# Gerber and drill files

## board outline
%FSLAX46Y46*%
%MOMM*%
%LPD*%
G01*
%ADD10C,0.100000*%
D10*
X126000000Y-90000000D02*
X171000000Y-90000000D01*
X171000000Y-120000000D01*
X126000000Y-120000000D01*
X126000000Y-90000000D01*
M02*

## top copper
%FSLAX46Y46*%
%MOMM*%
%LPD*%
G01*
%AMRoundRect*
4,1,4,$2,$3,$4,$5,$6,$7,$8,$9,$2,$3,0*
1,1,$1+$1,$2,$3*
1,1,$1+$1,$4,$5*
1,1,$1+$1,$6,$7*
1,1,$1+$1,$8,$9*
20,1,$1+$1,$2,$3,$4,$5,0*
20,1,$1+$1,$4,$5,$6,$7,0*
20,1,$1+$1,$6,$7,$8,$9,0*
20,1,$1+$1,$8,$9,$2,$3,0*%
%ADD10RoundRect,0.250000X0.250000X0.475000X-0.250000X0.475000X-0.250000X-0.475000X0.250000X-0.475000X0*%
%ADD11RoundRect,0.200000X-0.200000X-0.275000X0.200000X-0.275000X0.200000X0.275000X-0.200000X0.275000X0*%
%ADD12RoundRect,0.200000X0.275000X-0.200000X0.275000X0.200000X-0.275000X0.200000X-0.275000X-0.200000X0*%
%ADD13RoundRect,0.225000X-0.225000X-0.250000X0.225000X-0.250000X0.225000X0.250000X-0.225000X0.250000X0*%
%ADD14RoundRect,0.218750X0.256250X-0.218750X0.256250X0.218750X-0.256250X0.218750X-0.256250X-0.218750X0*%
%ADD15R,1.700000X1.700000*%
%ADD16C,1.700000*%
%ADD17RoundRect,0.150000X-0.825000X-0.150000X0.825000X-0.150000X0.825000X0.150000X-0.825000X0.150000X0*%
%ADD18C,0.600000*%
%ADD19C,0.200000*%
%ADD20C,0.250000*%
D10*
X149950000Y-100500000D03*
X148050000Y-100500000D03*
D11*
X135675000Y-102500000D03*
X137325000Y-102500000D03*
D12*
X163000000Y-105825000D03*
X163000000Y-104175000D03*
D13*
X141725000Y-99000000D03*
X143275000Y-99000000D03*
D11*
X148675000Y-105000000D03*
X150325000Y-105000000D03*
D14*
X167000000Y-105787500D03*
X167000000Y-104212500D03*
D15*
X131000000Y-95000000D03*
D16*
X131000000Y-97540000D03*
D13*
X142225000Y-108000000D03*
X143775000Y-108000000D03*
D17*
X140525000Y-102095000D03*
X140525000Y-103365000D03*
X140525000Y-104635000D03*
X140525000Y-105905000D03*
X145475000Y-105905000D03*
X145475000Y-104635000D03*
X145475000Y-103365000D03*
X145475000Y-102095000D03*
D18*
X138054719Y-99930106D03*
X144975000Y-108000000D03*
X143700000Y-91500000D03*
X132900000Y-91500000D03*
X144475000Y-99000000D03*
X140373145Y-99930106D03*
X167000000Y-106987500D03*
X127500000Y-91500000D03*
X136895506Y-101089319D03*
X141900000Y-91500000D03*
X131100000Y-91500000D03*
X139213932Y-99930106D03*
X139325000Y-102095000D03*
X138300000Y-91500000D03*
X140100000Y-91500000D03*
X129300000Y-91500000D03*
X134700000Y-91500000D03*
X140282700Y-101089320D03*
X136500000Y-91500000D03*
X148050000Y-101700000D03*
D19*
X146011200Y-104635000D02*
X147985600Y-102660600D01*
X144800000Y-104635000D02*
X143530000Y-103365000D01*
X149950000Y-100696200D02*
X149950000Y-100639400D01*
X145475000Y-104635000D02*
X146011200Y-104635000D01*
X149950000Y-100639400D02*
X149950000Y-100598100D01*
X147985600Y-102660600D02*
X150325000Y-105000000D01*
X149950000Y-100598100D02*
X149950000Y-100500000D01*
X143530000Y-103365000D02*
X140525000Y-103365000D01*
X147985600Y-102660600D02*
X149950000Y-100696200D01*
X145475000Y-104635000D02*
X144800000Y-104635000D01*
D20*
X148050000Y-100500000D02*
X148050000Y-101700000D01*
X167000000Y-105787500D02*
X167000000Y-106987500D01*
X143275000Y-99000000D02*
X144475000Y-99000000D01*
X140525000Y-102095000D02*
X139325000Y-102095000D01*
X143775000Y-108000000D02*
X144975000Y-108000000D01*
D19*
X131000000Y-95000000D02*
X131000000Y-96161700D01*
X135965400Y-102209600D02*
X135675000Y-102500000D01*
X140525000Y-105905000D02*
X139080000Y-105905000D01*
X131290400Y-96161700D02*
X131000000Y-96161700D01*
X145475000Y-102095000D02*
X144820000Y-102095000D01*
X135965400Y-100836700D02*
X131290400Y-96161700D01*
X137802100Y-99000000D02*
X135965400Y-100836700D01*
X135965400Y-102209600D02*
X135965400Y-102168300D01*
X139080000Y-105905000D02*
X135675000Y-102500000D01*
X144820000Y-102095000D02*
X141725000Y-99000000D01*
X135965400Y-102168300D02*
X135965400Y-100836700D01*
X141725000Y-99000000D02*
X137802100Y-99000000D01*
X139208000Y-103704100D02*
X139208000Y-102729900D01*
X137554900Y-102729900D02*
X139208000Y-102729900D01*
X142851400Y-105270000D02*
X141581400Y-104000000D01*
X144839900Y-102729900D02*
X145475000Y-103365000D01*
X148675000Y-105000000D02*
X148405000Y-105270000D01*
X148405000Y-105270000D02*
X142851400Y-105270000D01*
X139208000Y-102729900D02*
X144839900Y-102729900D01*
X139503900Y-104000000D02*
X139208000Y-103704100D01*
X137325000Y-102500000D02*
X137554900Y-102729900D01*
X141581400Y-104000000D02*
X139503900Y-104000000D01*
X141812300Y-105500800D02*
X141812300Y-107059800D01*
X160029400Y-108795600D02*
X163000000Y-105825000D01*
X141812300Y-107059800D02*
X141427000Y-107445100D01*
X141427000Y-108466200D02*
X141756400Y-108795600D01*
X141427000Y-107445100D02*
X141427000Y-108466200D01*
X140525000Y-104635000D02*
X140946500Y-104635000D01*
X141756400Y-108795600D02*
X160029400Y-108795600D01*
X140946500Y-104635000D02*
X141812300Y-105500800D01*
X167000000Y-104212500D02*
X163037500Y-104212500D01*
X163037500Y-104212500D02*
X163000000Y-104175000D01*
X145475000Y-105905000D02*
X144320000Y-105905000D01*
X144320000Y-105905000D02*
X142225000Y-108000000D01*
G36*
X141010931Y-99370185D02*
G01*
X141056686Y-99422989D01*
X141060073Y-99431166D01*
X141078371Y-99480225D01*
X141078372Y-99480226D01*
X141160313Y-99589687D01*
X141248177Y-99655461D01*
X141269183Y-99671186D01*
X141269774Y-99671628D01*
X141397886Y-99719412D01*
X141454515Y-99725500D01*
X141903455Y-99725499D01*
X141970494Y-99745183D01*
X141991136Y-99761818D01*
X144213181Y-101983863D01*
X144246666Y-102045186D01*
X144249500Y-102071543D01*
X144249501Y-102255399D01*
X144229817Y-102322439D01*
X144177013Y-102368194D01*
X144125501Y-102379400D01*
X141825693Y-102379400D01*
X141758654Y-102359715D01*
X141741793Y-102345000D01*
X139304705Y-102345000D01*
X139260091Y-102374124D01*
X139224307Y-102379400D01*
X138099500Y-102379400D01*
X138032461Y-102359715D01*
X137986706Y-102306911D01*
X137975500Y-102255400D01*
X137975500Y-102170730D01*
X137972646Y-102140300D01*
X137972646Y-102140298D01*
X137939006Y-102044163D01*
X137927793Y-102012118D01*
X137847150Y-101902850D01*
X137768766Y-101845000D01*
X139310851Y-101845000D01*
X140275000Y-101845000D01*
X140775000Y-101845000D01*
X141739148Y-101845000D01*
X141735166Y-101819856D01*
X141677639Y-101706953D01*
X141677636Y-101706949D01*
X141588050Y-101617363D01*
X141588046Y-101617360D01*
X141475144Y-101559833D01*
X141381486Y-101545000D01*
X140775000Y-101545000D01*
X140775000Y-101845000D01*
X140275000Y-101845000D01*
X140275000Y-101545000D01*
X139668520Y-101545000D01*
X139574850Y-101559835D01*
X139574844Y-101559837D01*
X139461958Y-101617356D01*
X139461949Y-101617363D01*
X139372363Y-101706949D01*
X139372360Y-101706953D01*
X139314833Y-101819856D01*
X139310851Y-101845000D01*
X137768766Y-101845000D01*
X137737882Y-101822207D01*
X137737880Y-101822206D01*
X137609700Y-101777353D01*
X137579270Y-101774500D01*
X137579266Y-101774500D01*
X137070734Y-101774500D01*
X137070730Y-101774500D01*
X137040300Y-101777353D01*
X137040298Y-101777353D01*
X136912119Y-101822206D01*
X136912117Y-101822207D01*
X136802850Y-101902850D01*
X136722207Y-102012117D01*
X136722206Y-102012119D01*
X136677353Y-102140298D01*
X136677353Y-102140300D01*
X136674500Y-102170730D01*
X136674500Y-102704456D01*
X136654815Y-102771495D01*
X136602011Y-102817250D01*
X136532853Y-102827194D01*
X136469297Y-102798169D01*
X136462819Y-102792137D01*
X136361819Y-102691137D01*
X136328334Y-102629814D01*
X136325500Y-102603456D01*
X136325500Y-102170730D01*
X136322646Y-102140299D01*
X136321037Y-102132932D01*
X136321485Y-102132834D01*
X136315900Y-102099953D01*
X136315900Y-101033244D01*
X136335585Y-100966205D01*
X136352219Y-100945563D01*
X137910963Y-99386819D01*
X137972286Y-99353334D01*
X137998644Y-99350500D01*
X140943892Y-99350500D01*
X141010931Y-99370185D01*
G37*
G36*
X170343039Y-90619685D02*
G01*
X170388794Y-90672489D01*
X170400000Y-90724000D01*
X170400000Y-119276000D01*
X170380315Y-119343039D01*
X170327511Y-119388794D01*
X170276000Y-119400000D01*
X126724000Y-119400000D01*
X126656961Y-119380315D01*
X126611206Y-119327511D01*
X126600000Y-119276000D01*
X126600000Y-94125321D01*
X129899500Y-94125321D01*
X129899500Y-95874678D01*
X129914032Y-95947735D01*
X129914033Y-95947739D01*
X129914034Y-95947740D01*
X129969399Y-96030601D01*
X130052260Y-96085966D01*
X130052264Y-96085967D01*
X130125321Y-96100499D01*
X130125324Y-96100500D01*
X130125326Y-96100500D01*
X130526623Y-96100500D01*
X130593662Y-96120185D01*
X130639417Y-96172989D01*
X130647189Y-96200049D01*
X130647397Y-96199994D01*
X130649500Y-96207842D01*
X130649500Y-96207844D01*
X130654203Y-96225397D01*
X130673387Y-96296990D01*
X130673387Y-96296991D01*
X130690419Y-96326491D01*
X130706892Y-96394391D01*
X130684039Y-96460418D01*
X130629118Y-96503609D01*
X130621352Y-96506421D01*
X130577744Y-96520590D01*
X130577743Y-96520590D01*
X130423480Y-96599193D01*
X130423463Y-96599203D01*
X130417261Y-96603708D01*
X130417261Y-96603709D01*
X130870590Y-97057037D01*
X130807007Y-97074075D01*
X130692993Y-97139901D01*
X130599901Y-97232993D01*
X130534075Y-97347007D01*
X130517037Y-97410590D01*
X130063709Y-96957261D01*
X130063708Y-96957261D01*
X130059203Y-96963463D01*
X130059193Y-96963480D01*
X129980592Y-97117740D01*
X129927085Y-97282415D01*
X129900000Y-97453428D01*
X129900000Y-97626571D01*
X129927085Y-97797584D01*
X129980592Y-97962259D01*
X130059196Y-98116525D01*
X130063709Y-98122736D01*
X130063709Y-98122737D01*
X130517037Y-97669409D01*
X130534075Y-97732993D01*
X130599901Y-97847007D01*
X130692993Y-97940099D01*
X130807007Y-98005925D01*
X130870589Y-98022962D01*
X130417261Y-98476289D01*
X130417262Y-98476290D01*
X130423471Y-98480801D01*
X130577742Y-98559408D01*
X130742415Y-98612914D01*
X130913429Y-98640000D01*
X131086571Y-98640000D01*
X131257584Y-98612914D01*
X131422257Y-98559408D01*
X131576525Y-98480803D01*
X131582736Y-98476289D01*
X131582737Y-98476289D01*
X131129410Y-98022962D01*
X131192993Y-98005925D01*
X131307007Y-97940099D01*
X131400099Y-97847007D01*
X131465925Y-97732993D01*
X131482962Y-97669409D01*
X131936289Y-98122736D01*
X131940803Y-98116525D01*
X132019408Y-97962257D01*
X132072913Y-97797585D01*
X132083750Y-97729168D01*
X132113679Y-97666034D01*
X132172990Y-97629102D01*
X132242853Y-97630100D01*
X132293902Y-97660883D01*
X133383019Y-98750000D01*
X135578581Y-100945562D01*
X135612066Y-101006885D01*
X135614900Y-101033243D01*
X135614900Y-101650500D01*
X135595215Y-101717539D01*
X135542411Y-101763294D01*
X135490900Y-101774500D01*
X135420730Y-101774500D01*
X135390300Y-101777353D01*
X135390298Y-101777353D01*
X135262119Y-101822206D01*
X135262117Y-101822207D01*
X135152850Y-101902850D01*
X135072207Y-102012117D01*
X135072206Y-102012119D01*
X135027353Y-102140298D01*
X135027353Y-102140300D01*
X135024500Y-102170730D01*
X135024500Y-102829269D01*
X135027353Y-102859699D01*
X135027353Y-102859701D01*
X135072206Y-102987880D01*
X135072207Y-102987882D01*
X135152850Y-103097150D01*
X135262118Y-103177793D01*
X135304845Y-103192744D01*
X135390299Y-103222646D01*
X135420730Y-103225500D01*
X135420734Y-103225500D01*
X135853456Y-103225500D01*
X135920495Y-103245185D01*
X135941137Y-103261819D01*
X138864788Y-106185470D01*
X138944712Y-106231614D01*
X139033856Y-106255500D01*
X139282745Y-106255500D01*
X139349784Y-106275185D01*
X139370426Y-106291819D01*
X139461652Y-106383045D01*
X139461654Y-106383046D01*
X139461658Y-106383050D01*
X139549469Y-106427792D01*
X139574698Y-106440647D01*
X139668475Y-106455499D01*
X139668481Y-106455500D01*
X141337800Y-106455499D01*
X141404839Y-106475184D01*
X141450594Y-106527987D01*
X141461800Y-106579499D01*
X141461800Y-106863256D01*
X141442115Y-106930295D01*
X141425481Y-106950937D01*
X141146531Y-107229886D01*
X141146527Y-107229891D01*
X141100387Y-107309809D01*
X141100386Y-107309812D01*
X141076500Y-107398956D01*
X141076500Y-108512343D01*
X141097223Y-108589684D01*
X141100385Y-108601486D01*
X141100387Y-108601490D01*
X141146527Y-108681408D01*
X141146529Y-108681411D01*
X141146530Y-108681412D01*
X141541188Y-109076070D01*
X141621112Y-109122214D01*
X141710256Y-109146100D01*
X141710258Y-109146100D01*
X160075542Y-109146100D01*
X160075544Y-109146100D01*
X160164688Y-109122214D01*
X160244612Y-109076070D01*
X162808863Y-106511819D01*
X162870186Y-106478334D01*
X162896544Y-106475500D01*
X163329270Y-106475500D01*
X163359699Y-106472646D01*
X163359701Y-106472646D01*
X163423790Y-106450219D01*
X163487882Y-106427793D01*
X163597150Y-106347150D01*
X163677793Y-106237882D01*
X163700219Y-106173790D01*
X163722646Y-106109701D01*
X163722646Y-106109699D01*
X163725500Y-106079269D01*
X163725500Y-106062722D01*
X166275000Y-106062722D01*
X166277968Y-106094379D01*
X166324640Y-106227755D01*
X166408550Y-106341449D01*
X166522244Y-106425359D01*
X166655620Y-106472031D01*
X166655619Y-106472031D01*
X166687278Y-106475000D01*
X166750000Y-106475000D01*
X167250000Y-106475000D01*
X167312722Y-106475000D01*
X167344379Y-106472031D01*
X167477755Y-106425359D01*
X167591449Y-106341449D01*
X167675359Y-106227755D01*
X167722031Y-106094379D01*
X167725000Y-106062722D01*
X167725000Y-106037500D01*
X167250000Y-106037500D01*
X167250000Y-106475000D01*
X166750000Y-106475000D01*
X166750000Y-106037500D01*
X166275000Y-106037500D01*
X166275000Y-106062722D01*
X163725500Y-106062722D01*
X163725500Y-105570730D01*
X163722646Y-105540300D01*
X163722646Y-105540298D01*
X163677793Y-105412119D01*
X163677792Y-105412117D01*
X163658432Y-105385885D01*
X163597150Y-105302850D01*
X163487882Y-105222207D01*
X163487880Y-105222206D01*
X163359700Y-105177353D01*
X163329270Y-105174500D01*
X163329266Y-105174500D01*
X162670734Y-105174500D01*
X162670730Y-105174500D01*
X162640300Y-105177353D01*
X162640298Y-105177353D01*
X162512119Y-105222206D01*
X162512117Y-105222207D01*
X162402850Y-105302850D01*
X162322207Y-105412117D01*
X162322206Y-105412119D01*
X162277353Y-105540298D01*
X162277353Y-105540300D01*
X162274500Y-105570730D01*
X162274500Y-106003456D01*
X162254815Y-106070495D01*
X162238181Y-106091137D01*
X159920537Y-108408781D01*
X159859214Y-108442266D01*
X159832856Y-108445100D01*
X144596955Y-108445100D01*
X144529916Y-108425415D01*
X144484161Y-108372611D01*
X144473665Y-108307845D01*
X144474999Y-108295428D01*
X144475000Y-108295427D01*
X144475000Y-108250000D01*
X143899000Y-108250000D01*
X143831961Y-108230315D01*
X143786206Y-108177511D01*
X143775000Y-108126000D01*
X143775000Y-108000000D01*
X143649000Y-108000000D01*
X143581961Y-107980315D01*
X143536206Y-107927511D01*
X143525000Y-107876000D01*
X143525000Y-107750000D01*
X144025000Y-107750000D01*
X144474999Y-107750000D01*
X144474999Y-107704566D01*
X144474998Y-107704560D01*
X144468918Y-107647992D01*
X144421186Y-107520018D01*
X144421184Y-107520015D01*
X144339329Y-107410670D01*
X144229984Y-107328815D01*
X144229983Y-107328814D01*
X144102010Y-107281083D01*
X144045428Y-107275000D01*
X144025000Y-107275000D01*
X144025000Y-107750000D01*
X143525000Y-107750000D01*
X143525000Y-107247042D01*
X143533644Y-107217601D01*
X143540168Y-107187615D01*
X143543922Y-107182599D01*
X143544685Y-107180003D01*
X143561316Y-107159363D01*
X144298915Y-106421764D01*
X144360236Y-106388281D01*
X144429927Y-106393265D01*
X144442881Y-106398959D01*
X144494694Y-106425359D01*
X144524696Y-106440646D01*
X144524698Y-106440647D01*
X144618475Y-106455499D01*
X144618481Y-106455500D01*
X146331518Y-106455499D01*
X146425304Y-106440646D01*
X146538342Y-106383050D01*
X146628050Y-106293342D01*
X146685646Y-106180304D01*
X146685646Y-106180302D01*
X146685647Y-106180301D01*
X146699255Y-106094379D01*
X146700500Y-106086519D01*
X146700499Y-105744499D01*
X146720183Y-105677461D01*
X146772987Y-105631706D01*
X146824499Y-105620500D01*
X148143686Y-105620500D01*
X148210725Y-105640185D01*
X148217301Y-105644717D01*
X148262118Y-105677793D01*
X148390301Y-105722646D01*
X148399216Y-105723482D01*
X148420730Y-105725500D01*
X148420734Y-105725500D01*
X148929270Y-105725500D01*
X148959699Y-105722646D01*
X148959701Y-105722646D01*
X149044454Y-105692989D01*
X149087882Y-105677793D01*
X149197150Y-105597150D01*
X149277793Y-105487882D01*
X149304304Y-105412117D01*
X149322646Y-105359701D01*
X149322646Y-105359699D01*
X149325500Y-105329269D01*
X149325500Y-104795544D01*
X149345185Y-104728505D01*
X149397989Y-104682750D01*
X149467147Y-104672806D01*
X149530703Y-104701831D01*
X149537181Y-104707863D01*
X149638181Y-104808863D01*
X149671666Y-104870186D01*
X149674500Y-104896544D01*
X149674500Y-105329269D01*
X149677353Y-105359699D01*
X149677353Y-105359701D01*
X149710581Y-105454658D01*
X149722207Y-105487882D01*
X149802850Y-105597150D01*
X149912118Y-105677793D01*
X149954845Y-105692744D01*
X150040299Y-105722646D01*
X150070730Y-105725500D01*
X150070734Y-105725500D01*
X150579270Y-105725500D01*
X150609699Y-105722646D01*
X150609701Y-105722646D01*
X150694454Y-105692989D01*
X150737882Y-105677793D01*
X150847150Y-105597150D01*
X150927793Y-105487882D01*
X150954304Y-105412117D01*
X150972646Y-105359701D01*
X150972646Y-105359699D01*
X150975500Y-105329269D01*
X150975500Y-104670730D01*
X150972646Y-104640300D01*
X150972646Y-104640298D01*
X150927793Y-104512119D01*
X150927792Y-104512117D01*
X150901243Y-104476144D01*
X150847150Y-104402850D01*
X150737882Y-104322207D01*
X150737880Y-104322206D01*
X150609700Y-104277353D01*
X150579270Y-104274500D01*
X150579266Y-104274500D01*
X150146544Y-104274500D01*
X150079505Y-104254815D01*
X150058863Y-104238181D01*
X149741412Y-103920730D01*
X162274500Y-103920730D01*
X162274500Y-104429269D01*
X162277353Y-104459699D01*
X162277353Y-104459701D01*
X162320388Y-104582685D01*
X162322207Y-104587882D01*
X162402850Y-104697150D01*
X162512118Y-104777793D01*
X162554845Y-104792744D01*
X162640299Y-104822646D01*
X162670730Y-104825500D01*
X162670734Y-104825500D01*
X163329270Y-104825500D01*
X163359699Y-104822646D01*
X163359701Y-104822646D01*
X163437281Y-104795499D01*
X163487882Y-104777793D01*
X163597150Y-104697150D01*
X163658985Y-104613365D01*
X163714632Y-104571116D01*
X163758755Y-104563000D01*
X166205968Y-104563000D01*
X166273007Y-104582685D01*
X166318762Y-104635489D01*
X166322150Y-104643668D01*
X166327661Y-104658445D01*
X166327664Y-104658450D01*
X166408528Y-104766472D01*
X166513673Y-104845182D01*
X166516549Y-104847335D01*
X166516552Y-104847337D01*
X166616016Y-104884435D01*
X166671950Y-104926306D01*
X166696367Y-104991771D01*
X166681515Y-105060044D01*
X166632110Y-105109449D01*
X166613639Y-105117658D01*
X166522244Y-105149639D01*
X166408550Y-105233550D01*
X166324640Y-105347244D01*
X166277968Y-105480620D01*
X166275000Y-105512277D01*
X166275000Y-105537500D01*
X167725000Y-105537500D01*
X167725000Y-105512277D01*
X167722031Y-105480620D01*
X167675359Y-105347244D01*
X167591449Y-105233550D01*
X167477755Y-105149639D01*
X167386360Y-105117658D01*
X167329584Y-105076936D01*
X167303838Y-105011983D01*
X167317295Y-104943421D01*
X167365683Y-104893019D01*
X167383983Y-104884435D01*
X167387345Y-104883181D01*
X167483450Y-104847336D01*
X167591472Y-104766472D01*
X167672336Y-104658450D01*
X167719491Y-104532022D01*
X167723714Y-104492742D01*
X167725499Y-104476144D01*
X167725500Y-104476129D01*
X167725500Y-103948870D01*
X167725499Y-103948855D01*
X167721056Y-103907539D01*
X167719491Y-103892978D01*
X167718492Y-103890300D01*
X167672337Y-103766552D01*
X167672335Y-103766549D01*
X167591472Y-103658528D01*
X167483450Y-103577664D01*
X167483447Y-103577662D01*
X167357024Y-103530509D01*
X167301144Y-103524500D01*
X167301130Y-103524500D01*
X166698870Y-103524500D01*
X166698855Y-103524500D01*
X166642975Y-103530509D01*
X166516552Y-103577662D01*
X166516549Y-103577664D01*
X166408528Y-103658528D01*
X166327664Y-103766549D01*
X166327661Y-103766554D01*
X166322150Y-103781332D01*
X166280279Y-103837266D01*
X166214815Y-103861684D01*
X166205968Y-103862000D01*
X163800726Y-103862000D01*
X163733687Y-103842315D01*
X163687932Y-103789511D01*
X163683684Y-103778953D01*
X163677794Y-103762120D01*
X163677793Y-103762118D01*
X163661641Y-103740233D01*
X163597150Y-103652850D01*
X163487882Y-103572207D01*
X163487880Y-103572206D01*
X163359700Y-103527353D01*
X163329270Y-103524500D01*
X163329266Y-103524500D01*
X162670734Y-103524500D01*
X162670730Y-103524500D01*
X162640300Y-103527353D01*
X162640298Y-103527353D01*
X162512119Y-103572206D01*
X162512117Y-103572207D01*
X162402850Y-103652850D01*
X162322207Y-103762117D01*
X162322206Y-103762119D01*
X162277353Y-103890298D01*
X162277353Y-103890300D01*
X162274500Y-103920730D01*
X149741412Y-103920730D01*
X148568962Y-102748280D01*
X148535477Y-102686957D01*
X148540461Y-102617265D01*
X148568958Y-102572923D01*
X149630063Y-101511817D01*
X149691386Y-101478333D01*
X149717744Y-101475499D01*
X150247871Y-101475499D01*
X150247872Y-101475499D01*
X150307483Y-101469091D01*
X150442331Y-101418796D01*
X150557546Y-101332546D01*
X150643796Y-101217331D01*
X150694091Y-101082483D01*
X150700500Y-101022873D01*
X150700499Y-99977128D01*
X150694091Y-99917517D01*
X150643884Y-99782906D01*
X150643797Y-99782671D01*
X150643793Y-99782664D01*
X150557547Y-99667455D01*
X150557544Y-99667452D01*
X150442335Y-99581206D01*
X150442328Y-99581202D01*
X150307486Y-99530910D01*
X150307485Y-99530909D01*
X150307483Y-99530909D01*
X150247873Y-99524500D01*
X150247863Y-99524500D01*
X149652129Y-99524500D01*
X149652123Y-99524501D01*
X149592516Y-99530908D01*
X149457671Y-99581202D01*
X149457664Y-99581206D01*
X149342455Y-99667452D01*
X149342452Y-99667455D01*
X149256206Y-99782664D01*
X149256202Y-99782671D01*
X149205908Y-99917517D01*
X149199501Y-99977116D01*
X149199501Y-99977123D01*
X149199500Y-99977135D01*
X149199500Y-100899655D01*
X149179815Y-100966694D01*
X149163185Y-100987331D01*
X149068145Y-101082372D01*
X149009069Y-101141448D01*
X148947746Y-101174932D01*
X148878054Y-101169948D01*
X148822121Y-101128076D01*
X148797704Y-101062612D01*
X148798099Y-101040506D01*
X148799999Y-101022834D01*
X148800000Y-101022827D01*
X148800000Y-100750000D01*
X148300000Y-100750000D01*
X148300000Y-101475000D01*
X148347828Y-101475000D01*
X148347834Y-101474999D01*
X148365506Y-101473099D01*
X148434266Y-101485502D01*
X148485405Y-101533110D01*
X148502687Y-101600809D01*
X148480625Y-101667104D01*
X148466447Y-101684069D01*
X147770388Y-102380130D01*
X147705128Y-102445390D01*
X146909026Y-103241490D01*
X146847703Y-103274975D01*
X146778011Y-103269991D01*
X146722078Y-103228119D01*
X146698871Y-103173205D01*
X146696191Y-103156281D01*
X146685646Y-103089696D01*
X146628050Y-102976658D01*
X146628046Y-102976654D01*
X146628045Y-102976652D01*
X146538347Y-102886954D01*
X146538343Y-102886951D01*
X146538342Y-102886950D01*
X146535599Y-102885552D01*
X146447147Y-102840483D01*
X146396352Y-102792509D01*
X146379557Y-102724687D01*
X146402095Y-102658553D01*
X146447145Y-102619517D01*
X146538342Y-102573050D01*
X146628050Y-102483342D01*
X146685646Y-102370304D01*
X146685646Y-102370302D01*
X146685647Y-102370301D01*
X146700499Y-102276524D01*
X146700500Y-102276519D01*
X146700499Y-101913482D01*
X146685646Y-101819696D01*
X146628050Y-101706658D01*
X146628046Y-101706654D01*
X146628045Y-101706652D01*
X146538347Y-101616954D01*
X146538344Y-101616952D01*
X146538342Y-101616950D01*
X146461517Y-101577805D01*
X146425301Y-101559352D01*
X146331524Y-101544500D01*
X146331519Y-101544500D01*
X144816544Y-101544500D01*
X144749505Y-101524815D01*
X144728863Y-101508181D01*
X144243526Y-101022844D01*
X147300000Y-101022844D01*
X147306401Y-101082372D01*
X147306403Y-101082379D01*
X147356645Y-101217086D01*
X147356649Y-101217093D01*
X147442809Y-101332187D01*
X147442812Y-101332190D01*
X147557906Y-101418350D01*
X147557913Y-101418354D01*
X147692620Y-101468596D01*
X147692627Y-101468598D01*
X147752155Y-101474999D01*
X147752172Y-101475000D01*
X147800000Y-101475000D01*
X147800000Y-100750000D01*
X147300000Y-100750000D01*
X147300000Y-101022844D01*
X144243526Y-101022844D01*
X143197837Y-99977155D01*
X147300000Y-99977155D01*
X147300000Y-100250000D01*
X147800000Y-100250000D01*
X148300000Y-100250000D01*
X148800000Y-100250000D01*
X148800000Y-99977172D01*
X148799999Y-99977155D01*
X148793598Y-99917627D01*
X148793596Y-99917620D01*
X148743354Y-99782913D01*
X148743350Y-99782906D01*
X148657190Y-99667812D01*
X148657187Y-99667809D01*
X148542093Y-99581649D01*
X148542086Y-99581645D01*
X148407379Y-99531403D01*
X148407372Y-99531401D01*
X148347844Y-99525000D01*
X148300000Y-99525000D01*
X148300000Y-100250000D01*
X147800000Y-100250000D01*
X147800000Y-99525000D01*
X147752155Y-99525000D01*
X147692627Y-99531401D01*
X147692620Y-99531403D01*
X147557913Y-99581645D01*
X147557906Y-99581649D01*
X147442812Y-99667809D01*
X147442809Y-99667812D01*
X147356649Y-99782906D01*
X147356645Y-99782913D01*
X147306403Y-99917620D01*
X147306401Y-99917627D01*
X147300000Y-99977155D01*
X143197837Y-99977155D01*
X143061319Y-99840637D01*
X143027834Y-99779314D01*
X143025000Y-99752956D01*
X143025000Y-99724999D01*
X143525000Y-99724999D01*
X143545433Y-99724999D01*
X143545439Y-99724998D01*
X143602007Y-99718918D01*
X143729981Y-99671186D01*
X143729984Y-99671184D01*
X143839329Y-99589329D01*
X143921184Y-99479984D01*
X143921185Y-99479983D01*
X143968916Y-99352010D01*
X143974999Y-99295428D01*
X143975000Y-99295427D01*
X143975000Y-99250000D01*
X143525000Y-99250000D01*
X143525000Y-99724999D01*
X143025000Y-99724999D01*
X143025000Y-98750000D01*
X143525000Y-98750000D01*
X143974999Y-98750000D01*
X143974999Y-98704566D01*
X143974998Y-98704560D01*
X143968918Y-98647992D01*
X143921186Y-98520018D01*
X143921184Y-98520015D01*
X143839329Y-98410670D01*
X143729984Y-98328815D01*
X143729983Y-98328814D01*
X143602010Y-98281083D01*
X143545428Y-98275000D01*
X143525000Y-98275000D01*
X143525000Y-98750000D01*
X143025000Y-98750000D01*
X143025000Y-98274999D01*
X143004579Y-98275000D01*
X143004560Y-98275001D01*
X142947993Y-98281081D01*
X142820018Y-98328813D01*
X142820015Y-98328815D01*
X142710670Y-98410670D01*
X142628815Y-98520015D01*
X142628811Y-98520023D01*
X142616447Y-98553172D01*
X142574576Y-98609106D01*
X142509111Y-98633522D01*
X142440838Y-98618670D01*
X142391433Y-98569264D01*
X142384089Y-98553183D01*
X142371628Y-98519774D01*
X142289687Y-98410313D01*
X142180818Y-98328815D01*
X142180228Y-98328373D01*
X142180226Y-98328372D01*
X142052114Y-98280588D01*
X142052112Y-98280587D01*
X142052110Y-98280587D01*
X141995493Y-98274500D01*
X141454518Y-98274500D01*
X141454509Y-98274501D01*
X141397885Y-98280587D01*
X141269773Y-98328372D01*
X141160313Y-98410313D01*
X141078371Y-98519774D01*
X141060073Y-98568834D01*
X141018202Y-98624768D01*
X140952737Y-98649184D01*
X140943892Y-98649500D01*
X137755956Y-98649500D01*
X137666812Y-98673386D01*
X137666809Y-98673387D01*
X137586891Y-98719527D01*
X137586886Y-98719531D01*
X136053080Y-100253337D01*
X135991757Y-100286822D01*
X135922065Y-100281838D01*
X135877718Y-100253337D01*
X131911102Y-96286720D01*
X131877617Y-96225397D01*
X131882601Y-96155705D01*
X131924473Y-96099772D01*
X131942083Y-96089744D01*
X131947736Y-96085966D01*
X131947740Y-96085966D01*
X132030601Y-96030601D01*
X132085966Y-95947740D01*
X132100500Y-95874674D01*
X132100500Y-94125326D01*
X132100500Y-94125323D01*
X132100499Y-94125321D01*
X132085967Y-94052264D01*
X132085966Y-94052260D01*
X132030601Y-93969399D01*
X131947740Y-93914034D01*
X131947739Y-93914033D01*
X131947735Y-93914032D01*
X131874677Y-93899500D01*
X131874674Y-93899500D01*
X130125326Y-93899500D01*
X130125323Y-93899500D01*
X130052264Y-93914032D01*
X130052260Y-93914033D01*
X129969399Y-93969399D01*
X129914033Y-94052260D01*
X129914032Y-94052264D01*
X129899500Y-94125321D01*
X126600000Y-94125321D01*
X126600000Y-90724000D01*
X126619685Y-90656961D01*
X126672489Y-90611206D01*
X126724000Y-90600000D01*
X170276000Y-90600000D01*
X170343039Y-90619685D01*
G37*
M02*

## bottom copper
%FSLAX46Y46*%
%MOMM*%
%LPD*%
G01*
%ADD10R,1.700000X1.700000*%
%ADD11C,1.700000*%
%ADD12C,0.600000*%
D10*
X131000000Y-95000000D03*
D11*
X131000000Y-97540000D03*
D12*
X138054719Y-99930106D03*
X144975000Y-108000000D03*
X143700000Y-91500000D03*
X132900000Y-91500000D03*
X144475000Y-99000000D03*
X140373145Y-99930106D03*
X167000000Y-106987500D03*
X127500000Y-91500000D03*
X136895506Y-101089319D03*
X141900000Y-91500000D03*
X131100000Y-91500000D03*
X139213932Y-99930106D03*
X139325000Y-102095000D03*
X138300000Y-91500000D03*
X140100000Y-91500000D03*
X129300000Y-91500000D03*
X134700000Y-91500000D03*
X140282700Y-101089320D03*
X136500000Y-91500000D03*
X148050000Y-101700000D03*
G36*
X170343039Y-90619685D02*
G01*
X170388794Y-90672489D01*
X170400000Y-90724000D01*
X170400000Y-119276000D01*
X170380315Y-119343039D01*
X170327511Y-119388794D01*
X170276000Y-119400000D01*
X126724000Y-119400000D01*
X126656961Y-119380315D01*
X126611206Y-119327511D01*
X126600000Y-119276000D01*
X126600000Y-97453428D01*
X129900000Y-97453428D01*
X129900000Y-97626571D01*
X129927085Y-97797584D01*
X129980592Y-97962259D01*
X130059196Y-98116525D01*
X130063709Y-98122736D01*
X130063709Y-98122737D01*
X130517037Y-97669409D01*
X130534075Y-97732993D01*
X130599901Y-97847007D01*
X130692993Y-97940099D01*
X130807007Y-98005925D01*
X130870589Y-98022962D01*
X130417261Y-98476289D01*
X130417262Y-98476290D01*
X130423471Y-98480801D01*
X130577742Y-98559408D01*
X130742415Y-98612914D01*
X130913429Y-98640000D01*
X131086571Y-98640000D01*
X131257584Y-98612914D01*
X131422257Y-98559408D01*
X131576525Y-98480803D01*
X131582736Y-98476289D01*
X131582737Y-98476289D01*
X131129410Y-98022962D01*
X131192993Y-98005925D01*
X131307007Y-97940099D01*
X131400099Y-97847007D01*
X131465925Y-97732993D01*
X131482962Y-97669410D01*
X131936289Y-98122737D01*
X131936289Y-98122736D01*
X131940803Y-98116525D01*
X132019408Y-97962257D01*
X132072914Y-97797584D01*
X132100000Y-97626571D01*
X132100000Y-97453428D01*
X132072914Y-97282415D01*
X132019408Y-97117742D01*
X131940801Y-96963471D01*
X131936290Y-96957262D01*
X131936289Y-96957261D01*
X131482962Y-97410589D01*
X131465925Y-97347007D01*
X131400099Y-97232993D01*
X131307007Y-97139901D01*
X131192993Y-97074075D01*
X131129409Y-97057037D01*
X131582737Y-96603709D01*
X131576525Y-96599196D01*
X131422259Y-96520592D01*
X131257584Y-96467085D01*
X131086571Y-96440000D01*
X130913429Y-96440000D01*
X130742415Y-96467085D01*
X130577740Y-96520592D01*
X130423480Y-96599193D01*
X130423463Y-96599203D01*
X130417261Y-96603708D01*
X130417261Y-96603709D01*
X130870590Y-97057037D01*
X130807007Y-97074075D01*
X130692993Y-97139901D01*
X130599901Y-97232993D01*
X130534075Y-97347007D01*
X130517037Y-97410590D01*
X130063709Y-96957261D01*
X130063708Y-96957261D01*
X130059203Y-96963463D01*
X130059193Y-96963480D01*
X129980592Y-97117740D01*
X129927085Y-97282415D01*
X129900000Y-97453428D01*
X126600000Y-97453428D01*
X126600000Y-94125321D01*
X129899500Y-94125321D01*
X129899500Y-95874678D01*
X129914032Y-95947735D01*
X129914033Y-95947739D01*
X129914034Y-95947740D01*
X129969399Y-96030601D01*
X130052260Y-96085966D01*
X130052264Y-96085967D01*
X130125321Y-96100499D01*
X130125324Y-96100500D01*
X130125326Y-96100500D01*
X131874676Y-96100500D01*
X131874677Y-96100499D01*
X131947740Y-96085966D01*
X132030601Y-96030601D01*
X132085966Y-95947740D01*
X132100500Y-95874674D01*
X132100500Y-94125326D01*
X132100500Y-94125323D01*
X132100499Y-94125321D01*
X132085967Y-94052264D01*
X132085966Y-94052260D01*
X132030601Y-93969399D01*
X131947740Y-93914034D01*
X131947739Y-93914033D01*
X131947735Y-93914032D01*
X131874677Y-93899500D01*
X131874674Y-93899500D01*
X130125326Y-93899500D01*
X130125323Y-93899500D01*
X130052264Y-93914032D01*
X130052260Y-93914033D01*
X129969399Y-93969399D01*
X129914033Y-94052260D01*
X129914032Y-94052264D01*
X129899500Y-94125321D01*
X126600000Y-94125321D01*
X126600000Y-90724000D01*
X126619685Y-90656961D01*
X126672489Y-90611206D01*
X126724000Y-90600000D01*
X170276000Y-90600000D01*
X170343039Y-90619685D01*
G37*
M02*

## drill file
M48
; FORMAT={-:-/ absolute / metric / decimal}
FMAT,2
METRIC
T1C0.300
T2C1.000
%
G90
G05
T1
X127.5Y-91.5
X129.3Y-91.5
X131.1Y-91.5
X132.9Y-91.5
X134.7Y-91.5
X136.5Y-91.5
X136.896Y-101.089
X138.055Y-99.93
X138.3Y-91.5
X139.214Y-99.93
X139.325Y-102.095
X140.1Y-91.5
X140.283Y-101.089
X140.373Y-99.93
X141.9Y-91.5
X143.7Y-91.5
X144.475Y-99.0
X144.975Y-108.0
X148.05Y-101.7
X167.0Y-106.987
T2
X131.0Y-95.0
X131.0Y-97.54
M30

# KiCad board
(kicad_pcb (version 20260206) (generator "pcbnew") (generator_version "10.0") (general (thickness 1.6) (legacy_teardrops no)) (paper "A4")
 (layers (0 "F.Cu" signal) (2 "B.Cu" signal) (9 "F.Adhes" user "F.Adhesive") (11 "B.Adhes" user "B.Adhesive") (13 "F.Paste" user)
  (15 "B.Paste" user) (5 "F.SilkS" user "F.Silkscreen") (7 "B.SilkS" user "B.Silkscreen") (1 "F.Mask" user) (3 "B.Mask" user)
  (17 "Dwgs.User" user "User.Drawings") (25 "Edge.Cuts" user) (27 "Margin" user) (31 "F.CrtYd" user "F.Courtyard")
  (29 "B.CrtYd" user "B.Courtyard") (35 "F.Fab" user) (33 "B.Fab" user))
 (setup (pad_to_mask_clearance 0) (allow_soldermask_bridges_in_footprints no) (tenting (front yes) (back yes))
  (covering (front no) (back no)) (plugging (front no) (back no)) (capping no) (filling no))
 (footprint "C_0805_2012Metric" (layer "F.Cu") (at 149 100.5 180)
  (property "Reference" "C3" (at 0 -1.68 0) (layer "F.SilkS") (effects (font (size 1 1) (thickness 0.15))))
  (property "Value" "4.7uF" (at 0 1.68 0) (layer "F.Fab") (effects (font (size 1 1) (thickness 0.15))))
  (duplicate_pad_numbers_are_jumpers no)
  (pad "1" smd roundrect (at -0.95 0 180) (size 1 1.45) (layers "F.Cu" "F.Mask" "F.Paste") (roundrect_rratio 0.25) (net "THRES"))
  (pad "2" smd roundrect (at 0.95 0 180) (size 1 1.45) (layers "F.Cu" "F.Mask" "F.Paste") (roundrect_rratio 0.25) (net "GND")))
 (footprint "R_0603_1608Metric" (layer "F.Cu") (at 136.5 102.5)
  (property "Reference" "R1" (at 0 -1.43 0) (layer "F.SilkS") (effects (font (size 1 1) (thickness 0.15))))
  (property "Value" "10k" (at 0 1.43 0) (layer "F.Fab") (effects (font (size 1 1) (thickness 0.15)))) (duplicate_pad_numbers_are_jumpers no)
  (pad "1" smd roundrect (at -0.825 0) (size 0.8 0.95) (layers "F.Cu" "F.Mask" "F.Paste") (roundrect_rratio 0.25) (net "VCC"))
  (pad "2" smd roundrect (at 0.825 0) (size 0.8 0.95) (layers "F.Cu" "F.Mask" "F.Paste") (roundrect_rratio 0.25) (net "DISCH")))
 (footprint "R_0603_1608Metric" (layer "F.Cu") (at 163 105 90)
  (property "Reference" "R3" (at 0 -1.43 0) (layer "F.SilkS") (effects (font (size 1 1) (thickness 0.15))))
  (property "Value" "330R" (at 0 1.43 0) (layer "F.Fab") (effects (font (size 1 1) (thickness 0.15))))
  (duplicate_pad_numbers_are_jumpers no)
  (pad "1" smd roundrect (at -0.825 0 90) (size 0.8 0.95) (layers "F.Cu" "F.Mask" "F.Paste") (roundrect_rratio 0.25) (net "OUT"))
  (pad "2" smd roundrect (at 0.825 0 90) (size 0.8 0.95) (layers "F.Cu" "F.Mask" "F.Paste") (roundrect_rratio 0.25) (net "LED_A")))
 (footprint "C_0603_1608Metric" (layer "F.Cu") (at 142.5 99)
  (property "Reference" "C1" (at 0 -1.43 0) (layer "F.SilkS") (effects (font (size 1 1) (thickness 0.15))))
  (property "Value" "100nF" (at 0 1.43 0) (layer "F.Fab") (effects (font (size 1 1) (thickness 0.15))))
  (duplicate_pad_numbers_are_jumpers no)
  (pad "1" smd roundrect (at -0.775 0) (size 0.9 0.95) (layers "F.Cu" "F.Mask" "F.Paste") (roundrect_rratio 0.25) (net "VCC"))
  (pad "2" smd roundrect (at 0.775 0) (size 0.9 0.95) (layers "F.Cu" "F.Mask" "F.Paste") (roundrect_rratio 0.25) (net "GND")))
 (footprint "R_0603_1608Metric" (layer "F.Cu") (at 149.5 105)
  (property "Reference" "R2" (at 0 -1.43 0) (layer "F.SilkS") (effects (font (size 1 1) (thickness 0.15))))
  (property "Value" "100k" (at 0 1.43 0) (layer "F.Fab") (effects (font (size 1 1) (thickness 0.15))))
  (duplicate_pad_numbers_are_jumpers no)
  (pad "1" smd roundrect (at -0.825 0) (size 0.8 0.95) (layers "F.Cu" "F.Mask" "F.Paste") (roundrect_rratio 0.25) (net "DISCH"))
  (pad "2" smd roundrect (at 0.825 0) (size 0.8 0.95) (layers "F.Cu" "F.Mask" "F.Paste") (roundrect_rratio 0.25) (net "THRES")))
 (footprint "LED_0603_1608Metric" (layer "F.Cu") (at 167 105 90)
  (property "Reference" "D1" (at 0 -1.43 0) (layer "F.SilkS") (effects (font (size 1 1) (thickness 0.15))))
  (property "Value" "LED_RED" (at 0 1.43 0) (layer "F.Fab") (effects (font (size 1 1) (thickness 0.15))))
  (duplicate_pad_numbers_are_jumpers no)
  (pad "1" smd roundrect (at -0.7875 0 90) (size 0.875 0.95) (layers "F.Cu" "F.Mask" "F.Paste") (roundrect_rratio 0.25) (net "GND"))
  (pad "2" smd roundrect (at 0.7875 0 90) (size 0.875 0.95) (layers "F.Cu" "F.Mask" "F.Paste") (roundrect_rratio 0.25) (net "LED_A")))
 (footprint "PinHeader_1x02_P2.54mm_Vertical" (layer "F.Cu") (at 131 95)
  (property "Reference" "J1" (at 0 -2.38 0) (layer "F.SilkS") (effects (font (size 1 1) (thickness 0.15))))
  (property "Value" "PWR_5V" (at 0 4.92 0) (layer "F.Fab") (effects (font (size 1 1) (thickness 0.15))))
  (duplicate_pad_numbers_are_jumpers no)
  (pad "1" thru_hole rect (at 0 0) (size 1.7 1.7) (drill 1) (layers "*.Cu" "*.Mask") (remove_unused_layers no) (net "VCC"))
  (pad "2" thru_hole circle (at 0 2.54) (size 1.7 1.7) (drill 1) (layers "*.Cu" "*.Mask") (remove_unused_layers no) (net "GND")))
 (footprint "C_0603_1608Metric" (layer "F.Cu") (at 143 108)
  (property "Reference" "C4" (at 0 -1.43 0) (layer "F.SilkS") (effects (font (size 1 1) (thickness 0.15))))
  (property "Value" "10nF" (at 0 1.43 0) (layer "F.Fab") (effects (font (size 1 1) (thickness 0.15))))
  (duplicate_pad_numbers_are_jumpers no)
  (pad "1" smd roundrect (at -0.775 0) (size 0.9 0.95) (layers "F.Cu" "F.Mask" "F.Paste") (roundrect_rratio 0.25) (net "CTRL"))
  (pad "2" smd roundrect (at 0.775 0) (size 0.9 0.95) (layers "F.Cu" "F.Mask" "F.Paste") (roundrect_rratio 0.25) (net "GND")))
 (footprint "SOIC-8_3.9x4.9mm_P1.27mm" (layer "F.Cu") (at 143 104)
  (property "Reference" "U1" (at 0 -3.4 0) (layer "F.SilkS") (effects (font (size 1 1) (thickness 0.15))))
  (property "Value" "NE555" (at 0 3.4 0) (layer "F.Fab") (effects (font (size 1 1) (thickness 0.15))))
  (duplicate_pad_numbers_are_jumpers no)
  (pad "1" smd roundrect (at -2.475 -1.905) (size 1.95 0.6) (layers "F.Cu" "F.Mask" "F.Paste") (roundrect_rratio 0.25) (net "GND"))
  (pad "2" smd roundrect (at -2.475 -0.635) (size 1.95 0.6) (layers "F.Cu" "F.Mask" "F.Paste") (roundrect_rratio 0.25) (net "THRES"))
  (pad "3" smd roundrect (at -2.475 0.635) (size 1.95 0.6) (layers "F.Cu" "F.Mask" "F.Paste") (roundrect_rratio 0.25) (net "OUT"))
  (pad "4" smd roundrect (at -2.475 1.905) (size 1.95 0.6) (layers "F.Cu" "F.Mask" "F.Paste") (roundrect_rratio 0.25) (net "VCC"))
  (pad "5" smd roundrect (at 2.475 1.905) (size 1.95 0.6) (layers "F.Cu" "F.Mask" "F.Paste") (roundrect_rratio 0.25) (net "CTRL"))
  (pad "6" smd roundrect (at 2.475 0.635) (size 1.95 0.6) (layers "F.Cu" "F.Mask" "F.Paste") (roundrect_rratio 0.25) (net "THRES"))
  (pad "7" smd roundrect (at 2.475 -0.635) (size 1.95 0.6) (layers "F.Cu" "F.Mask" "F.Paste") (roundrect_rratio 0.25) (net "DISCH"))
  (pad "8" smd roundrect (at 2.475 -1.905) (size 1.95 0.6) (layers "F.Cu" "F.Mask" "F.Paste") (roundrect_rratio 0.25) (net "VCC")))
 (gr_rect (start 126 90) (end 171 120) (stroke (width 0.1) (type default)) (fill no) (layer "Edge.Cuts"))
 (segment (start 146.0112 104.635) (end 147.9856 102.6606) (width 0.2) (layer "F.Cu") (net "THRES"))
 (segment (start 144.8 104.635) (end 143.53 103.365) (width 0.2) (layer "F.Cu") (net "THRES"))
 (segment (start 149.95 100.6962) (end 149.95 100.6394) (width 0.2) (layer "F.Cu") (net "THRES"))
 (segment (start 145.475 104.635) (end 146.0112 104.635) (width 0.2) (layer "F.Cu") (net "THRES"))
 (segment (start 149.95 100.6394) (end 149.95 100.5981) (width 0.2) (layer "F.Cu") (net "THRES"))
 (segment (start 147.9856 102.6606) (end 150.325 105) (width 0.2) (layer "F.Cu") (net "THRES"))
 (segment (start 149.95 100.5981) (end 149.95 100.5) (width 0.2) (layer "F.Cu") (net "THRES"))
 (segment (start 143.53 103.365) (end 140.525 103.365) (width 0.2) (layer "F.Cu") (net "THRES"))
 (segment (start 147.9856 102.6606) (end 149.95 100.6962) (width 0.2) (layer "F.Cu") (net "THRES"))
 (segment (start 145.475 104.635) (end 144.8 104.635) (width 0.2) (layer "F.Cu") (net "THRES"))
 (segment (start 148.05 100.5) (end 148.05 101.7) (width 0.25) (layer "F.Cu") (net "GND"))
 (segment (start 167 105.7875) (end 167 106.9875) (width 0.25) (layer "F.Cu") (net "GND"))
 (segment (start 143.275 99) (end 144.475 99) (width 0.25) (layer "F.Cu") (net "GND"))
 (segment (start 140.525 102.095) (end 139.325 102.095) (width 0.25) (layer "F.Cu") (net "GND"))
 (segment (start 143.775 108) (end 144.975 108) (width 0.25) (layer "F.Cu") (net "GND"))
 (via (at 138.054719 99.930106) (size 0.6) (drill 0.3) (layers "F.Cu" "B.Cu") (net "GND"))
 (via (at 144.975 108) (size 0.6) (drill 0.3) (layers "F.Cu" "B.Cu") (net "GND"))
 (via (at 143.7 91.5) (size 0.6) (drill 0.3) (layers "F.Cu" "B.Cu") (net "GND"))
 (via (at 132.9 91.5) (size 0.6) (drill 0.3) (layers "F.Cu" "B.Cu") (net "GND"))
 (via (at 144.475 99) (size 0.6) (drill 0.3) (layers "F.Cu" "B.Cu") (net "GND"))
 (via (at 140.373145 99.930106) (size 0.6) (drill 0.3) (layers "F.Cu" "B.Cu") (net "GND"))
 (via (at 167 106.9875) (size 0.6) (drill 0.3) (layers "F.Cu" "B.Cu") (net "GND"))
 (via (at 127.5 91.5) (size 0.6) (drill 0.3) (layers "F.Cu" "B.Cu") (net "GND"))
 (via (at 136.895506 101.089319) (size 0.6) (drill 0.3) (layers "F.Cu" "B.Cu") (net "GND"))
 (via (at 141.9 91.5) (size 0.6) (drill 0.3) (layers "F.Cu" "B.Cu") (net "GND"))
 (via (at 131.1 91.5) (size 0.6) (drill 0.3) (layers "F.Cu" "B.Cu") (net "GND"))
 (via (at 139.213932 99.930106) (size 0.6) (drill 0.3) (layers "F.Cu" "B.Cu") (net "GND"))
 (via (at 139.325 102.095) (size 0.6) (drill 0.3) (layers "F.Cu" "B.Cu") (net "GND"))
 (via (at 138.3 91.5) (size 0.6) (drill 0.3) (layers "F.Cu" "B.Cu") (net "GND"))
 (via (at 140.1 91.5) (size 0.6) (drill 0.3) (layers "F.Cu" "B.Cu") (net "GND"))
 (via (at 129.3 91.5) (size 0.6) (drill 0.3) (layers "F.Cu" "B.Cu") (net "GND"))
 (via (at 134.7 91.5) (size 0.6) (drill 0.3) (layers "F.Cu" "B.Cu") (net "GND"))
 (via (at 140.2827 101.08932) (size 0.6) (drill 0.3) (layers "F.Cu" "B.Cu") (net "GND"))
 (via (at 136.5 91.5) (size 0.6) (drill 0.3) (layers "F.Cu" "B.Cu") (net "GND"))
 (via (at 148.05 101.7) (size 0.6) (drill 0.3) (layers "F.Cu" "B.Cu") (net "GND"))
 (segment (start 131 95) (end 131 96.1617) (width 0.2) (layer "F.Cu") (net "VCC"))
 (segment (start 135.9654 102.2096) (end 135.675 102.5) (width 0.2) (layer "F.Cu") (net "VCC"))
 (segment (start 140.525 105.905) (end 139.08 105.905) (width 0.2) (layer "F.Cu") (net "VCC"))
 (segment (start 131.2904 96.1617) (end 131 96.1617) (width 0.2) (layer "F.Cu") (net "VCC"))
 (segment (start 145.475 102.095) (end 144.82 102.095) (width 0.2) (layer "F.Cu") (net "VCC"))
 (segment (start 135.9654 100.8367) (end 131.2904 96.1617) (width 0.2) (layer "F.Cu") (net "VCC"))
 (segment (start 137.8021 99) (end 135.9654 100.8367) (width 0.2) (layer "F.Cu") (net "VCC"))
 (segment (start 135.9654 102.2096) (end 135.9654 102.1683) (width 0.2) (layer "F.Cu") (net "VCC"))
 (segment (start 139.08 105.905) (end 135.675 102.5) (width 0.2) (layer "F.Cu") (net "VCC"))
 (segment (start 144.82 102.095) (end 141.725 99) (width 0.2) (layer "F.Cu") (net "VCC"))
 (segment (start 135.9654 102.1683) (end 135.9654 100.8367) (width 0.2) (layer "F.Cu") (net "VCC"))
 (segment (start 141.725 99) (end 137.8021 99) (width 0.2) (layer "F.Cu") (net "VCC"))
 (segment (start 139.208 103.7041) (end 139.208 102.7299) (width 0.2) (layer "F.Cu") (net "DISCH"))
 (segment (start 137.5549 102.7299) (end 139.208 102.7299) (width 0.2) (layer "F.Cu") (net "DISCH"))
 (segment (start 142.8514 105.27) (end 141.5814 104) (width 0.2) (layer "F.Cu") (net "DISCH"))
 (segment (start 144.8399 102.7299) (end 145.475 103.365) (width 0.2) (layer "F.Cu") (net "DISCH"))
 (segment (start 148.675 105) (end 148.405 105.27) (width 0.2) (layer "F.Cu") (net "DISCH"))
 (segment (start 148.405 105.27) (end 142.8514 105.27) (width 0.2) (layer "F.Cu") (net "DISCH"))
 (segment (start 139.208 102.7299) (end 144.8399 102.7299) (width 0.2) (layer "F.Cu") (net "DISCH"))
 (segment (start 139.5039 104) (end 139.208 103.7041) (width 0.2) (layer "F.Cu") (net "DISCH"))
 (segment (start 137.325 102.5) (end 137.5549 102.7299) (width 0.2) (layer "F.Cu") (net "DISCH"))
 (segment (start 141.5814 104) (end 139.5039 104) (width 0.2) (layer "F.Cu") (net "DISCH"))
 (segment (start 141.8123 105.5008) (end 141.8123 107.0598) (width 0.2) (layer "F.Cu") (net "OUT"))
 (segment (start 160.0294 108.7956) (end 163 105.825) (width 0.2) (layer "F.Cu") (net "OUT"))
 (segment (start 141.8123 107.0598) (end 141.427 107.4451) (width 0.2) (layer "F.Cu") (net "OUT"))
 (segment (start 141.427 108.4662) (end 141.7564 108.7956) (width 0.2) (layer "F.Cu") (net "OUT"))
 (segment (start 141.427 107.4451) (end 141.427 108.4662) (width 0.2) (layer "F.Cu") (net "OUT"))
 (segment (start 140.525 104.635) (end 140.9465 104.635) (width 0.2) (layer "F.Cu") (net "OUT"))
 (segment (start 141.7564 108.7956) (end 160.0294 108.7956) (width 0.2) (layer "F.Cu") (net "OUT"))
 (segment (start 140.9465 104.635) (end 141.8123 105.5008) (width 0.2) (layer "F.Cu") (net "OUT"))
 (segment (start 167 104.2125) (end 163.0375 104.2125) (width 0.2) (layer "F.Cu") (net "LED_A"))
 (segment (start 163.0375 104.2125) (end 163 104.175) (width 0.2) (layer "F.Cu") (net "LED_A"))
 (segment (start 145.475 105.905) (end 144.32 105.905) (width 0.2) (layer "F.Cu") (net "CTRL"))
 (segment (start 144.32 105.905) (end 142.225 108) (width 0.2) (layer "F.Cu") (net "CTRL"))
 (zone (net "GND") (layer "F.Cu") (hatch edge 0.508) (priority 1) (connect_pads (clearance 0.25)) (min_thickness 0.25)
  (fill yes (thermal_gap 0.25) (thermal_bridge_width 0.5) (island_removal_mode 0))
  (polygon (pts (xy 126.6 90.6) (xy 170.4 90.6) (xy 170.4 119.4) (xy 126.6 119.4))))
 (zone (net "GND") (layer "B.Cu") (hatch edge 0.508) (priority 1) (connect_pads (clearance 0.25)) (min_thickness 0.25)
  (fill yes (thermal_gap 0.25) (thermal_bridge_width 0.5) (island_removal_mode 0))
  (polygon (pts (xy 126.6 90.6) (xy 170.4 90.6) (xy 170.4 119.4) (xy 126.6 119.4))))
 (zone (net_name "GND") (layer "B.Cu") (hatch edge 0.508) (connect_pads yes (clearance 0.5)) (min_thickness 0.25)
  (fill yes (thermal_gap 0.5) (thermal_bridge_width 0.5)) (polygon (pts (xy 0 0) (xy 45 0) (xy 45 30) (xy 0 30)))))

